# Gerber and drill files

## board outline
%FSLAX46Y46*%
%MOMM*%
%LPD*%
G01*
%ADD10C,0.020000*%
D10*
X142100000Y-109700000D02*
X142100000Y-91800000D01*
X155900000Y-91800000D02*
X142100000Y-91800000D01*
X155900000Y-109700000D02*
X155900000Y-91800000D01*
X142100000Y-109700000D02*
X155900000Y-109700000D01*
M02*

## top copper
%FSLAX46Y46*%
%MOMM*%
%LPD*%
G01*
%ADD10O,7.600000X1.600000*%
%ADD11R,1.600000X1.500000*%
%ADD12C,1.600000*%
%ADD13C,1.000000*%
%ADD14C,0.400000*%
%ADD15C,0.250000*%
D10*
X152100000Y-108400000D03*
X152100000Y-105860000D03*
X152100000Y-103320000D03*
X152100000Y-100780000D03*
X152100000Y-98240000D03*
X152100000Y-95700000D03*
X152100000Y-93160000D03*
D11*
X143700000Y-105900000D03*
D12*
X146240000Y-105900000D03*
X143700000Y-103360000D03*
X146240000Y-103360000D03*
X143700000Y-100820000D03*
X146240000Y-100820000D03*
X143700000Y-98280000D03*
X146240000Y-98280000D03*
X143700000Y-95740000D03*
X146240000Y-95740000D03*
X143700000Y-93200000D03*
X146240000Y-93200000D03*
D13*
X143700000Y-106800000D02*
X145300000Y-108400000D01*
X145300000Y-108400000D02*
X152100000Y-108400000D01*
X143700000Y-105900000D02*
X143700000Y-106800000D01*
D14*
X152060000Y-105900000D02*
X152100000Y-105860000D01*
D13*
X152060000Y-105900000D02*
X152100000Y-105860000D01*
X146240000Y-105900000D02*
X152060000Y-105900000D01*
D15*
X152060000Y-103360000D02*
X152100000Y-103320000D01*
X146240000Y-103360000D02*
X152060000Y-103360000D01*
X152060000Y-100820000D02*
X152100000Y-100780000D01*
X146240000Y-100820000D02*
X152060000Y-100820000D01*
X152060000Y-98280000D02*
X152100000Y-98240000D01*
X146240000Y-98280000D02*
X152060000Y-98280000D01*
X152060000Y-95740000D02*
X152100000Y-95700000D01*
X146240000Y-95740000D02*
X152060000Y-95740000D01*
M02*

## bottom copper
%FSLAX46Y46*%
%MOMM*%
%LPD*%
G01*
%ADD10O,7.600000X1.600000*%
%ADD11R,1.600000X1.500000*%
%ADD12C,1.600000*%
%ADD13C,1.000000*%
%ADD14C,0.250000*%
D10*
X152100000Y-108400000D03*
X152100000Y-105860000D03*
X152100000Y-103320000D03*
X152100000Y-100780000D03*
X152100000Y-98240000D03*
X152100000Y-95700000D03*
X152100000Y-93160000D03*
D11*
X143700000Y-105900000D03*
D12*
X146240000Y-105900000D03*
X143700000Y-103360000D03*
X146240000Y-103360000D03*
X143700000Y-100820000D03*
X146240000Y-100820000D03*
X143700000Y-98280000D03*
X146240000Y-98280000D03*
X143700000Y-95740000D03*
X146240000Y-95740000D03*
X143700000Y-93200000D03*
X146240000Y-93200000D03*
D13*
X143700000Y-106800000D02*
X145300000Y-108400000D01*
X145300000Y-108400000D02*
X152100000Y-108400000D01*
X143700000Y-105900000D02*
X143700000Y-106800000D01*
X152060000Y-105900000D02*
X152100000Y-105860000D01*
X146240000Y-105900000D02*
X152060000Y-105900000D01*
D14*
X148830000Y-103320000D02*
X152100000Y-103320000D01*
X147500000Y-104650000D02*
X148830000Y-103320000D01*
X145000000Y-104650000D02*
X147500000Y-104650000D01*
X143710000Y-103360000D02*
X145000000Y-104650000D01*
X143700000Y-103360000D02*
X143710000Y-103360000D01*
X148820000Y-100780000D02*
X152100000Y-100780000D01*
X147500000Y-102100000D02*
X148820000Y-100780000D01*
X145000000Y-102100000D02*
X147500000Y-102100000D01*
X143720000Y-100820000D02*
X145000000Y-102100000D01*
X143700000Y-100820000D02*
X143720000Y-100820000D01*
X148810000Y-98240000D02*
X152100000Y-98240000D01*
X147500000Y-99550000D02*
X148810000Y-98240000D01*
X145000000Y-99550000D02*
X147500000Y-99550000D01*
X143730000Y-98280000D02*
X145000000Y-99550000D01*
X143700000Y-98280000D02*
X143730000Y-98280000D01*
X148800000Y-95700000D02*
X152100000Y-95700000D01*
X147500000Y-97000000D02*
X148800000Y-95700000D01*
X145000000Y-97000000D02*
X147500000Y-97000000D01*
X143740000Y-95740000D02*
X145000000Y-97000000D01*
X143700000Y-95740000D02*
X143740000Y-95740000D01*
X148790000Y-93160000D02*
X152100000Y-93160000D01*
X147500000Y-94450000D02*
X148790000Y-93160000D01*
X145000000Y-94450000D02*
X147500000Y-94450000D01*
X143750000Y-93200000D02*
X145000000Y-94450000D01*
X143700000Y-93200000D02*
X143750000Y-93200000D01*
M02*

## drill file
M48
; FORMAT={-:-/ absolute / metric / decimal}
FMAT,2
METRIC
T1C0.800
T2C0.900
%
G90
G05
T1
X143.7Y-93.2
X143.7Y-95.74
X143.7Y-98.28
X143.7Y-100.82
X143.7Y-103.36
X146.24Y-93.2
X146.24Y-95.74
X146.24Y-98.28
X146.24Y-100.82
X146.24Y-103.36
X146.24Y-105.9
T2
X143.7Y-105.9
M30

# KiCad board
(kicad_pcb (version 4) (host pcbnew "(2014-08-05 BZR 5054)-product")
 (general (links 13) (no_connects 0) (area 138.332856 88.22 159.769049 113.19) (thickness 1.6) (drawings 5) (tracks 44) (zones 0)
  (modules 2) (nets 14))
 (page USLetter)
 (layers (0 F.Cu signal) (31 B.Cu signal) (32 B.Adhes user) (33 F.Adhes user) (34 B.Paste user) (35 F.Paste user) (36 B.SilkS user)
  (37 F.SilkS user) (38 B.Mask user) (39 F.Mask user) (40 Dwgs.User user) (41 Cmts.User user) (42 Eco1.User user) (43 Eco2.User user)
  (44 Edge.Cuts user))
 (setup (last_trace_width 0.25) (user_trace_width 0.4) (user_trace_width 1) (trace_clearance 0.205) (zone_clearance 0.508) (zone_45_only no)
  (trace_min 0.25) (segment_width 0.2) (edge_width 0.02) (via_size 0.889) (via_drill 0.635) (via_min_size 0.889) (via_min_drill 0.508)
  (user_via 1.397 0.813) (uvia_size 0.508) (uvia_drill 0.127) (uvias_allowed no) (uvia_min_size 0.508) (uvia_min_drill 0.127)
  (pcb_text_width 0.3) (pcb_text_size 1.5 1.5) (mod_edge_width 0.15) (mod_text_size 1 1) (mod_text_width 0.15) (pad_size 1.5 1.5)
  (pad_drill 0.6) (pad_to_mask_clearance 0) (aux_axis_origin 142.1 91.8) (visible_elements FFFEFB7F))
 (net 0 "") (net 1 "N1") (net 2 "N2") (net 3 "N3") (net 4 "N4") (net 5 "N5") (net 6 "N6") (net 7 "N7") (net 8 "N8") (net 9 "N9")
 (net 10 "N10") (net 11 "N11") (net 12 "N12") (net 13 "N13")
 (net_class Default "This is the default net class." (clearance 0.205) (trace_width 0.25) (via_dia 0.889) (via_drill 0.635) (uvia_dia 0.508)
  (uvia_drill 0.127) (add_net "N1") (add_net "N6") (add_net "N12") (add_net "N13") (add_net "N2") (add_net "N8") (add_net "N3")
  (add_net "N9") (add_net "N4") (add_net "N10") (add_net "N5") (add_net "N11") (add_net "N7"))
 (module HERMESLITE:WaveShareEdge (layer F.Cu) (at 152.1 108.4 180)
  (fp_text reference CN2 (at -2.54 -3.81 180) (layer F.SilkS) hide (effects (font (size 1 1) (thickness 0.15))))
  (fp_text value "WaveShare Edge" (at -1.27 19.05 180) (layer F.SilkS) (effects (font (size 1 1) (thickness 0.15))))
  (pad 1 smd oval (at 0 0 180) (size 7.6 1.6) (layers F.Cu F.Paste F.Mask) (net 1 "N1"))
  (pad 3 smd oval (at 0 2.54 180) (size 7.6 1.6) (layers F.Cu F.Paste F.Mask) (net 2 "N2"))
  (pad 5 smd oval (at 0 5.08 180) (size 7.6 1.6) (layers F.Cu F.Paste F.Mask) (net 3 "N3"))
  (pad 7 smd oval (at 0 7.62 180) (size 7.6 1.6) (layers F.Cu F.Paste F.Mask) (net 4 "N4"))
  (pad 9 smd oval (at 0 10.16 180) (size 7.6 1.6) (layers F.Cu F.Paste F.Mask) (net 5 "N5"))
  (pad 11 smd oval (at 0 12.7 180) (size 7.6 1.6) (layers F.Cu F.Paste F.Mask) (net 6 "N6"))
  (pad 13 smd oval (at 0 15.24 180) (size 7.6 1.6) (layers F.Cu F.Paste F.Mask) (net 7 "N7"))
  (pad 2 smd oval (at 0 0 180) (size 7.6 1.6) (layers B.Cu B.Paste B.Mask) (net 1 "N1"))
  (pad 4 smd oval (at 0 2.54 180) (size 7.6 1.6) (layers B.Cu B.Paste B.Mask) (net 2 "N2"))
  (pad 6 smd oval (at 0 5.08 180) (size 7.6 1.6) (layers B.Cu B.Paste B.Mask) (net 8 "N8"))
  (pad 8 smd oval (at 0 7.62 180) (size 7.6 1.6) (layers B.Cu B.Paste B.Mask) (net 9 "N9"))
  (pad 10 smd oval (at 0 10.16 180) (size 7.6 1.6) (layers B.Cu B.Paste B.Mask) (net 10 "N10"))
  (pad 12 smd oval (at 0 12.7 180) (size 7.6 1.6) (layers B.Cu B.Paste B.Mask) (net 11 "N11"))
  (pad 14 smd oval (at 0 15.24 180) (size 7.6 1.6) (layers B.Cu B.Paste B.Mask) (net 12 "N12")))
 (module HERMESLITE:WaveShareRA (layer F.Cu) (at 143.7 105.9)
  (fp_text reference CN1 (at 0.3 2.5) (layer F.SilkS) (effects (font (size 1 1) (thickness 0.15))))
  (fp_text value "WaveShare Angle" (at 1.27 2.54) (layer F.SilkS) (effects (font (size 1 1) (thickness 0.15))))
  (pad 1 thru_hole rect (at 0 0) (size 1.6 1.5) (drill 0.9) (layers *.Cu *.Mask F.SilkS) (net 1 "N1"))
  (pad 2 thru_hole circle (at 2.54 0) (size 1.6 1.6) (drill 0.8) (layers *.Cu *.Mask F.SilkS) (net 2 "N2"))
  (pad 3 thru_hole circle (at 0 -2.54) (size 1.6 1.6) (drill 0.8) (layers *.Cu *.Mask F.SilkS) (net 8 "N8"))
  (pad 4 thru_hole circle (at 2.54 -2.54) (size 1.6 1.6) (drill 0.8) (layers *.Cu *.Mask F.SilkS) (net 3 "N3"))
  (pad 5 thru_hole circle (at 0 -5.08) (size 1.6 1.6) (drill 0.8) (layers *.Cu *.Mask F.SilkS) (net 9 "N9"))
  (pad 6 thru_hole circle (at 2.54 -5.08) (size 1.6 1.6) (drill 0.8) (layers *.Cu *.Mask F.SilkS) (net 4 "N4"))
  (pad 7 thru_hole circle (at 0 -7.62) (size 1.6 1.6) (drill 0.8) (layers *.Cu *.Mask F.SilkS) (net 10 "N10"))
  (pad 8 thru_hole circle (at 2.54 -7.62) (size 1.6 1.6) (drill 0.8) (layers *.Cu *.Mask F.SilkS) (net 5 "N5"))
  (pad 9 thru_hole circle (at 0 -10.16) (size 1.6 1.6) (drill 0.8) (layers *.Cu *.Mask F.SilkS) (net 11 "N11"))
  (pad 10 thru_hole circle (at 2.54 -10.16) (size 1.6 1.6) (drill 0.8) (layers *.Cu *.Mask F.SilkS) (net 6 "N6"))
  (pad 11 thru_hole circle (at 0 -12.7) (size 1.6 1.6) (drill 0.8) (layers *.Cu *.Mask F.SilkS) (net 12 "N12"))
  (pad 12 thru_hole circle (at 2.54 -12.7) (size 1.6 1.6) (drill 0.8) (layers *.Cu *.Mask F.SilkS) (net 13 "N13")))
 (gr_line (start 142.1 109.7) (end 142.1 91.8) (angle 90) (layer Edge.Cuts) (width 0.02))
 (gr_line (start 155.9 91.8) (end 142.1 91.8) (angle 90) (layer Edge.Cuts) (width 0.02))
 (gr_line (start 155.9 109.7) (end 155.9 91.8) (angle 90) (layer Edge.Cuts) (width 0.02))
 (gr_line (start 142.1 109.7) (end 155.9 109.7) (angle 90) (layer Edge.Cuts) (width 0.02))
 (segment (start 143.7 106.8) (end 145.3 108.4) (width 1) (layer B.Cu) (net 1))
 (segment (start 145.3 108.4) (end 152.1 108.4) (width 1) (layer B.Cu) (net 1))
 (segment (start 143.7 105.9) (end 143.7 106.8) (width 1) (layer B.Cu) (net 1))
 (segment (start 143.7 106.8) (end 145.3 108.4) (width 1) (layer F.Cu) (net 1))
 (segment (start 145.3 108.4) (end 152.1 108.4) (width 1) (layer F.Cu) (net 1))
 (segment (start 143.7 105.9) (end 143.7 106.8) (width 1) (layer F.Cu) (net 1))
 (segment (start 152.06 105.9) (end 152.1 105.86) (width 0.4) (layer F.Cu) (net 2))
 (segment (start 152.06 105.9) (end 152.1 105.86) (width 1) (layer F.Cu) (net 2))
 (segment (start 146.24 105.9) (end 152.06 105.9) (width 1) (layer F.Cu) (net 2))
 (segment (start 152.06 105.9) (end 152.1 105.86) (width 1) (layer B.Cu) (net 2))
 (segment (start 146.24 105.9) (end 152.06 105.9) (width 1) (layer B.Cu) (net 2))
 (segment (start 148.83 103.32) (end 152.1 103.32) (width 0.25) (layer B.Cu) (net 8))
 (segment (start 147.5 104.65) (end 148.83 103.32) (width 0.25) (layer B.Cu) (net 8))
 (segment (start 145 104.65) (end 147.5 104.65) (width 0.25) (layer B.Cu) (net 8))
 (segment (start 143.71 103.36) (end 145 104.65) (width 0.25) (layer B.Cu) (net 8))
 (segment (start 143.7 103.36) (end 143.71 103.36) (width 0.25) (layer B.Cu) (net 8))
 (segment (start 152.06 103.36) (end 152.1 103.32) (width 0.25) (layer F.Cu) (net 3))
 (segment (start 146.24 103.36) (end 152.06 103.36) (width 0.25) (layer F.Cu) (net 3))
 (segment (start 148.82 100.78) (end 152.1 100.78) (width 0.25) (layer B.Cu) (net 9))
 (segment (start 147.5 102.1) (end 148.82 100.78) (width 0.25) (layer B.Cu) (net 9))
 (segment (start 145 102.1) (end 147.5 102.1) (width 0.25) (layer B.Cu) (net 9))
 (segment (start 143.72 100.82) (end 145 102.1) (width 0.25) (layer B.Cu) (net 9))
 (segment (start 143.7 100.82) (end 143.72 100.82) (width 0.25) (layer B.Cu) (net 9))
 (segment (start 152.06 100.82) (end 152.1 100.78) (width 0.25) (layer F.Cu) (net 4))
 (segment (start 146.24 100.82) (end 152.06 100.82) (width 0.25) (layer F.Cu) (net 4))
 (segment (start 148.81 98.24) (end 152.1 98.24) (width 0.25) (layer B.Cu) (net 10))
 (segment (start 147.5 99.55) (end 148.81 98.24) (width 0.25) (layer B.Cu) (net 10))
 (segment (start 145 99.55) (end 147.5 99.55) (width 0.25) (layer B.Cu) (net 10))
 (segment (start 143.73 98.28) (end 145 99.55) (width 0.25) (layer B.Cu) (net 10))
 (segment (start 143.7 98.28) (end 143.73 98.28) (width 0.25) (layer B.Cu) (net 10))
 (segment (start 152.06 98.28) (end 152.1 98.24) (width 0.25) (layer F.Cu) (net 5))
 (segment (start 146.24 98.28) (end 152.06 98.28) (width 0.25) (layer F.Cu) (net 5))
 (segment (start 148.8 95.7) (end 152.1 95.7) (width 0.25) (layer B.Cu) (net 11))
 (segment (start 147.5 97) (end 148.8 95.7) (width 0.25) (layer B.Cu) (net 11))
 (segment (start 145 97) (end 147.5 97) (width 0.25) (layer B.Cu) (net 11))
 (segment (start 143.74 95.74) (end 145 97) (width 0.25) (layer B.Cu) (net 11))
 (segment (start 143.7 95.74) (end 143.74 95.74) (width 0.25) (layer B.Cu) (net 11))
 (segment (start 152.06 95.74) (end 152.1 95.7) (width 0.25) (layer F.Cu) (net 6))
 (segment (start 146.24 95.74) (end 152.06 95.74) (width 0.25) (layer F.Cu) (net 6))
 (segment (start 148.79 93.16) (end 152.1 93.16) (width 0.25) (layer B.Cu) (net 12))
 (segment (start 147.5 94.45) (end 148.79 93.16) (width 0.25) (layer B.Cu) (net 12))
 (segment (start 145 94.45) (end 147.5 94.45) (width 0.25) (layer B.Cu) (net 12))
 (segment (start 143.75 93.2) (end 145 94.45) (width 0.25) (layer B.Cu) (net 12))
 (segment (start 143.7 93.2) (end 143.75 93.2) (width 0.25) (layer B.Cu) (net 12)))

